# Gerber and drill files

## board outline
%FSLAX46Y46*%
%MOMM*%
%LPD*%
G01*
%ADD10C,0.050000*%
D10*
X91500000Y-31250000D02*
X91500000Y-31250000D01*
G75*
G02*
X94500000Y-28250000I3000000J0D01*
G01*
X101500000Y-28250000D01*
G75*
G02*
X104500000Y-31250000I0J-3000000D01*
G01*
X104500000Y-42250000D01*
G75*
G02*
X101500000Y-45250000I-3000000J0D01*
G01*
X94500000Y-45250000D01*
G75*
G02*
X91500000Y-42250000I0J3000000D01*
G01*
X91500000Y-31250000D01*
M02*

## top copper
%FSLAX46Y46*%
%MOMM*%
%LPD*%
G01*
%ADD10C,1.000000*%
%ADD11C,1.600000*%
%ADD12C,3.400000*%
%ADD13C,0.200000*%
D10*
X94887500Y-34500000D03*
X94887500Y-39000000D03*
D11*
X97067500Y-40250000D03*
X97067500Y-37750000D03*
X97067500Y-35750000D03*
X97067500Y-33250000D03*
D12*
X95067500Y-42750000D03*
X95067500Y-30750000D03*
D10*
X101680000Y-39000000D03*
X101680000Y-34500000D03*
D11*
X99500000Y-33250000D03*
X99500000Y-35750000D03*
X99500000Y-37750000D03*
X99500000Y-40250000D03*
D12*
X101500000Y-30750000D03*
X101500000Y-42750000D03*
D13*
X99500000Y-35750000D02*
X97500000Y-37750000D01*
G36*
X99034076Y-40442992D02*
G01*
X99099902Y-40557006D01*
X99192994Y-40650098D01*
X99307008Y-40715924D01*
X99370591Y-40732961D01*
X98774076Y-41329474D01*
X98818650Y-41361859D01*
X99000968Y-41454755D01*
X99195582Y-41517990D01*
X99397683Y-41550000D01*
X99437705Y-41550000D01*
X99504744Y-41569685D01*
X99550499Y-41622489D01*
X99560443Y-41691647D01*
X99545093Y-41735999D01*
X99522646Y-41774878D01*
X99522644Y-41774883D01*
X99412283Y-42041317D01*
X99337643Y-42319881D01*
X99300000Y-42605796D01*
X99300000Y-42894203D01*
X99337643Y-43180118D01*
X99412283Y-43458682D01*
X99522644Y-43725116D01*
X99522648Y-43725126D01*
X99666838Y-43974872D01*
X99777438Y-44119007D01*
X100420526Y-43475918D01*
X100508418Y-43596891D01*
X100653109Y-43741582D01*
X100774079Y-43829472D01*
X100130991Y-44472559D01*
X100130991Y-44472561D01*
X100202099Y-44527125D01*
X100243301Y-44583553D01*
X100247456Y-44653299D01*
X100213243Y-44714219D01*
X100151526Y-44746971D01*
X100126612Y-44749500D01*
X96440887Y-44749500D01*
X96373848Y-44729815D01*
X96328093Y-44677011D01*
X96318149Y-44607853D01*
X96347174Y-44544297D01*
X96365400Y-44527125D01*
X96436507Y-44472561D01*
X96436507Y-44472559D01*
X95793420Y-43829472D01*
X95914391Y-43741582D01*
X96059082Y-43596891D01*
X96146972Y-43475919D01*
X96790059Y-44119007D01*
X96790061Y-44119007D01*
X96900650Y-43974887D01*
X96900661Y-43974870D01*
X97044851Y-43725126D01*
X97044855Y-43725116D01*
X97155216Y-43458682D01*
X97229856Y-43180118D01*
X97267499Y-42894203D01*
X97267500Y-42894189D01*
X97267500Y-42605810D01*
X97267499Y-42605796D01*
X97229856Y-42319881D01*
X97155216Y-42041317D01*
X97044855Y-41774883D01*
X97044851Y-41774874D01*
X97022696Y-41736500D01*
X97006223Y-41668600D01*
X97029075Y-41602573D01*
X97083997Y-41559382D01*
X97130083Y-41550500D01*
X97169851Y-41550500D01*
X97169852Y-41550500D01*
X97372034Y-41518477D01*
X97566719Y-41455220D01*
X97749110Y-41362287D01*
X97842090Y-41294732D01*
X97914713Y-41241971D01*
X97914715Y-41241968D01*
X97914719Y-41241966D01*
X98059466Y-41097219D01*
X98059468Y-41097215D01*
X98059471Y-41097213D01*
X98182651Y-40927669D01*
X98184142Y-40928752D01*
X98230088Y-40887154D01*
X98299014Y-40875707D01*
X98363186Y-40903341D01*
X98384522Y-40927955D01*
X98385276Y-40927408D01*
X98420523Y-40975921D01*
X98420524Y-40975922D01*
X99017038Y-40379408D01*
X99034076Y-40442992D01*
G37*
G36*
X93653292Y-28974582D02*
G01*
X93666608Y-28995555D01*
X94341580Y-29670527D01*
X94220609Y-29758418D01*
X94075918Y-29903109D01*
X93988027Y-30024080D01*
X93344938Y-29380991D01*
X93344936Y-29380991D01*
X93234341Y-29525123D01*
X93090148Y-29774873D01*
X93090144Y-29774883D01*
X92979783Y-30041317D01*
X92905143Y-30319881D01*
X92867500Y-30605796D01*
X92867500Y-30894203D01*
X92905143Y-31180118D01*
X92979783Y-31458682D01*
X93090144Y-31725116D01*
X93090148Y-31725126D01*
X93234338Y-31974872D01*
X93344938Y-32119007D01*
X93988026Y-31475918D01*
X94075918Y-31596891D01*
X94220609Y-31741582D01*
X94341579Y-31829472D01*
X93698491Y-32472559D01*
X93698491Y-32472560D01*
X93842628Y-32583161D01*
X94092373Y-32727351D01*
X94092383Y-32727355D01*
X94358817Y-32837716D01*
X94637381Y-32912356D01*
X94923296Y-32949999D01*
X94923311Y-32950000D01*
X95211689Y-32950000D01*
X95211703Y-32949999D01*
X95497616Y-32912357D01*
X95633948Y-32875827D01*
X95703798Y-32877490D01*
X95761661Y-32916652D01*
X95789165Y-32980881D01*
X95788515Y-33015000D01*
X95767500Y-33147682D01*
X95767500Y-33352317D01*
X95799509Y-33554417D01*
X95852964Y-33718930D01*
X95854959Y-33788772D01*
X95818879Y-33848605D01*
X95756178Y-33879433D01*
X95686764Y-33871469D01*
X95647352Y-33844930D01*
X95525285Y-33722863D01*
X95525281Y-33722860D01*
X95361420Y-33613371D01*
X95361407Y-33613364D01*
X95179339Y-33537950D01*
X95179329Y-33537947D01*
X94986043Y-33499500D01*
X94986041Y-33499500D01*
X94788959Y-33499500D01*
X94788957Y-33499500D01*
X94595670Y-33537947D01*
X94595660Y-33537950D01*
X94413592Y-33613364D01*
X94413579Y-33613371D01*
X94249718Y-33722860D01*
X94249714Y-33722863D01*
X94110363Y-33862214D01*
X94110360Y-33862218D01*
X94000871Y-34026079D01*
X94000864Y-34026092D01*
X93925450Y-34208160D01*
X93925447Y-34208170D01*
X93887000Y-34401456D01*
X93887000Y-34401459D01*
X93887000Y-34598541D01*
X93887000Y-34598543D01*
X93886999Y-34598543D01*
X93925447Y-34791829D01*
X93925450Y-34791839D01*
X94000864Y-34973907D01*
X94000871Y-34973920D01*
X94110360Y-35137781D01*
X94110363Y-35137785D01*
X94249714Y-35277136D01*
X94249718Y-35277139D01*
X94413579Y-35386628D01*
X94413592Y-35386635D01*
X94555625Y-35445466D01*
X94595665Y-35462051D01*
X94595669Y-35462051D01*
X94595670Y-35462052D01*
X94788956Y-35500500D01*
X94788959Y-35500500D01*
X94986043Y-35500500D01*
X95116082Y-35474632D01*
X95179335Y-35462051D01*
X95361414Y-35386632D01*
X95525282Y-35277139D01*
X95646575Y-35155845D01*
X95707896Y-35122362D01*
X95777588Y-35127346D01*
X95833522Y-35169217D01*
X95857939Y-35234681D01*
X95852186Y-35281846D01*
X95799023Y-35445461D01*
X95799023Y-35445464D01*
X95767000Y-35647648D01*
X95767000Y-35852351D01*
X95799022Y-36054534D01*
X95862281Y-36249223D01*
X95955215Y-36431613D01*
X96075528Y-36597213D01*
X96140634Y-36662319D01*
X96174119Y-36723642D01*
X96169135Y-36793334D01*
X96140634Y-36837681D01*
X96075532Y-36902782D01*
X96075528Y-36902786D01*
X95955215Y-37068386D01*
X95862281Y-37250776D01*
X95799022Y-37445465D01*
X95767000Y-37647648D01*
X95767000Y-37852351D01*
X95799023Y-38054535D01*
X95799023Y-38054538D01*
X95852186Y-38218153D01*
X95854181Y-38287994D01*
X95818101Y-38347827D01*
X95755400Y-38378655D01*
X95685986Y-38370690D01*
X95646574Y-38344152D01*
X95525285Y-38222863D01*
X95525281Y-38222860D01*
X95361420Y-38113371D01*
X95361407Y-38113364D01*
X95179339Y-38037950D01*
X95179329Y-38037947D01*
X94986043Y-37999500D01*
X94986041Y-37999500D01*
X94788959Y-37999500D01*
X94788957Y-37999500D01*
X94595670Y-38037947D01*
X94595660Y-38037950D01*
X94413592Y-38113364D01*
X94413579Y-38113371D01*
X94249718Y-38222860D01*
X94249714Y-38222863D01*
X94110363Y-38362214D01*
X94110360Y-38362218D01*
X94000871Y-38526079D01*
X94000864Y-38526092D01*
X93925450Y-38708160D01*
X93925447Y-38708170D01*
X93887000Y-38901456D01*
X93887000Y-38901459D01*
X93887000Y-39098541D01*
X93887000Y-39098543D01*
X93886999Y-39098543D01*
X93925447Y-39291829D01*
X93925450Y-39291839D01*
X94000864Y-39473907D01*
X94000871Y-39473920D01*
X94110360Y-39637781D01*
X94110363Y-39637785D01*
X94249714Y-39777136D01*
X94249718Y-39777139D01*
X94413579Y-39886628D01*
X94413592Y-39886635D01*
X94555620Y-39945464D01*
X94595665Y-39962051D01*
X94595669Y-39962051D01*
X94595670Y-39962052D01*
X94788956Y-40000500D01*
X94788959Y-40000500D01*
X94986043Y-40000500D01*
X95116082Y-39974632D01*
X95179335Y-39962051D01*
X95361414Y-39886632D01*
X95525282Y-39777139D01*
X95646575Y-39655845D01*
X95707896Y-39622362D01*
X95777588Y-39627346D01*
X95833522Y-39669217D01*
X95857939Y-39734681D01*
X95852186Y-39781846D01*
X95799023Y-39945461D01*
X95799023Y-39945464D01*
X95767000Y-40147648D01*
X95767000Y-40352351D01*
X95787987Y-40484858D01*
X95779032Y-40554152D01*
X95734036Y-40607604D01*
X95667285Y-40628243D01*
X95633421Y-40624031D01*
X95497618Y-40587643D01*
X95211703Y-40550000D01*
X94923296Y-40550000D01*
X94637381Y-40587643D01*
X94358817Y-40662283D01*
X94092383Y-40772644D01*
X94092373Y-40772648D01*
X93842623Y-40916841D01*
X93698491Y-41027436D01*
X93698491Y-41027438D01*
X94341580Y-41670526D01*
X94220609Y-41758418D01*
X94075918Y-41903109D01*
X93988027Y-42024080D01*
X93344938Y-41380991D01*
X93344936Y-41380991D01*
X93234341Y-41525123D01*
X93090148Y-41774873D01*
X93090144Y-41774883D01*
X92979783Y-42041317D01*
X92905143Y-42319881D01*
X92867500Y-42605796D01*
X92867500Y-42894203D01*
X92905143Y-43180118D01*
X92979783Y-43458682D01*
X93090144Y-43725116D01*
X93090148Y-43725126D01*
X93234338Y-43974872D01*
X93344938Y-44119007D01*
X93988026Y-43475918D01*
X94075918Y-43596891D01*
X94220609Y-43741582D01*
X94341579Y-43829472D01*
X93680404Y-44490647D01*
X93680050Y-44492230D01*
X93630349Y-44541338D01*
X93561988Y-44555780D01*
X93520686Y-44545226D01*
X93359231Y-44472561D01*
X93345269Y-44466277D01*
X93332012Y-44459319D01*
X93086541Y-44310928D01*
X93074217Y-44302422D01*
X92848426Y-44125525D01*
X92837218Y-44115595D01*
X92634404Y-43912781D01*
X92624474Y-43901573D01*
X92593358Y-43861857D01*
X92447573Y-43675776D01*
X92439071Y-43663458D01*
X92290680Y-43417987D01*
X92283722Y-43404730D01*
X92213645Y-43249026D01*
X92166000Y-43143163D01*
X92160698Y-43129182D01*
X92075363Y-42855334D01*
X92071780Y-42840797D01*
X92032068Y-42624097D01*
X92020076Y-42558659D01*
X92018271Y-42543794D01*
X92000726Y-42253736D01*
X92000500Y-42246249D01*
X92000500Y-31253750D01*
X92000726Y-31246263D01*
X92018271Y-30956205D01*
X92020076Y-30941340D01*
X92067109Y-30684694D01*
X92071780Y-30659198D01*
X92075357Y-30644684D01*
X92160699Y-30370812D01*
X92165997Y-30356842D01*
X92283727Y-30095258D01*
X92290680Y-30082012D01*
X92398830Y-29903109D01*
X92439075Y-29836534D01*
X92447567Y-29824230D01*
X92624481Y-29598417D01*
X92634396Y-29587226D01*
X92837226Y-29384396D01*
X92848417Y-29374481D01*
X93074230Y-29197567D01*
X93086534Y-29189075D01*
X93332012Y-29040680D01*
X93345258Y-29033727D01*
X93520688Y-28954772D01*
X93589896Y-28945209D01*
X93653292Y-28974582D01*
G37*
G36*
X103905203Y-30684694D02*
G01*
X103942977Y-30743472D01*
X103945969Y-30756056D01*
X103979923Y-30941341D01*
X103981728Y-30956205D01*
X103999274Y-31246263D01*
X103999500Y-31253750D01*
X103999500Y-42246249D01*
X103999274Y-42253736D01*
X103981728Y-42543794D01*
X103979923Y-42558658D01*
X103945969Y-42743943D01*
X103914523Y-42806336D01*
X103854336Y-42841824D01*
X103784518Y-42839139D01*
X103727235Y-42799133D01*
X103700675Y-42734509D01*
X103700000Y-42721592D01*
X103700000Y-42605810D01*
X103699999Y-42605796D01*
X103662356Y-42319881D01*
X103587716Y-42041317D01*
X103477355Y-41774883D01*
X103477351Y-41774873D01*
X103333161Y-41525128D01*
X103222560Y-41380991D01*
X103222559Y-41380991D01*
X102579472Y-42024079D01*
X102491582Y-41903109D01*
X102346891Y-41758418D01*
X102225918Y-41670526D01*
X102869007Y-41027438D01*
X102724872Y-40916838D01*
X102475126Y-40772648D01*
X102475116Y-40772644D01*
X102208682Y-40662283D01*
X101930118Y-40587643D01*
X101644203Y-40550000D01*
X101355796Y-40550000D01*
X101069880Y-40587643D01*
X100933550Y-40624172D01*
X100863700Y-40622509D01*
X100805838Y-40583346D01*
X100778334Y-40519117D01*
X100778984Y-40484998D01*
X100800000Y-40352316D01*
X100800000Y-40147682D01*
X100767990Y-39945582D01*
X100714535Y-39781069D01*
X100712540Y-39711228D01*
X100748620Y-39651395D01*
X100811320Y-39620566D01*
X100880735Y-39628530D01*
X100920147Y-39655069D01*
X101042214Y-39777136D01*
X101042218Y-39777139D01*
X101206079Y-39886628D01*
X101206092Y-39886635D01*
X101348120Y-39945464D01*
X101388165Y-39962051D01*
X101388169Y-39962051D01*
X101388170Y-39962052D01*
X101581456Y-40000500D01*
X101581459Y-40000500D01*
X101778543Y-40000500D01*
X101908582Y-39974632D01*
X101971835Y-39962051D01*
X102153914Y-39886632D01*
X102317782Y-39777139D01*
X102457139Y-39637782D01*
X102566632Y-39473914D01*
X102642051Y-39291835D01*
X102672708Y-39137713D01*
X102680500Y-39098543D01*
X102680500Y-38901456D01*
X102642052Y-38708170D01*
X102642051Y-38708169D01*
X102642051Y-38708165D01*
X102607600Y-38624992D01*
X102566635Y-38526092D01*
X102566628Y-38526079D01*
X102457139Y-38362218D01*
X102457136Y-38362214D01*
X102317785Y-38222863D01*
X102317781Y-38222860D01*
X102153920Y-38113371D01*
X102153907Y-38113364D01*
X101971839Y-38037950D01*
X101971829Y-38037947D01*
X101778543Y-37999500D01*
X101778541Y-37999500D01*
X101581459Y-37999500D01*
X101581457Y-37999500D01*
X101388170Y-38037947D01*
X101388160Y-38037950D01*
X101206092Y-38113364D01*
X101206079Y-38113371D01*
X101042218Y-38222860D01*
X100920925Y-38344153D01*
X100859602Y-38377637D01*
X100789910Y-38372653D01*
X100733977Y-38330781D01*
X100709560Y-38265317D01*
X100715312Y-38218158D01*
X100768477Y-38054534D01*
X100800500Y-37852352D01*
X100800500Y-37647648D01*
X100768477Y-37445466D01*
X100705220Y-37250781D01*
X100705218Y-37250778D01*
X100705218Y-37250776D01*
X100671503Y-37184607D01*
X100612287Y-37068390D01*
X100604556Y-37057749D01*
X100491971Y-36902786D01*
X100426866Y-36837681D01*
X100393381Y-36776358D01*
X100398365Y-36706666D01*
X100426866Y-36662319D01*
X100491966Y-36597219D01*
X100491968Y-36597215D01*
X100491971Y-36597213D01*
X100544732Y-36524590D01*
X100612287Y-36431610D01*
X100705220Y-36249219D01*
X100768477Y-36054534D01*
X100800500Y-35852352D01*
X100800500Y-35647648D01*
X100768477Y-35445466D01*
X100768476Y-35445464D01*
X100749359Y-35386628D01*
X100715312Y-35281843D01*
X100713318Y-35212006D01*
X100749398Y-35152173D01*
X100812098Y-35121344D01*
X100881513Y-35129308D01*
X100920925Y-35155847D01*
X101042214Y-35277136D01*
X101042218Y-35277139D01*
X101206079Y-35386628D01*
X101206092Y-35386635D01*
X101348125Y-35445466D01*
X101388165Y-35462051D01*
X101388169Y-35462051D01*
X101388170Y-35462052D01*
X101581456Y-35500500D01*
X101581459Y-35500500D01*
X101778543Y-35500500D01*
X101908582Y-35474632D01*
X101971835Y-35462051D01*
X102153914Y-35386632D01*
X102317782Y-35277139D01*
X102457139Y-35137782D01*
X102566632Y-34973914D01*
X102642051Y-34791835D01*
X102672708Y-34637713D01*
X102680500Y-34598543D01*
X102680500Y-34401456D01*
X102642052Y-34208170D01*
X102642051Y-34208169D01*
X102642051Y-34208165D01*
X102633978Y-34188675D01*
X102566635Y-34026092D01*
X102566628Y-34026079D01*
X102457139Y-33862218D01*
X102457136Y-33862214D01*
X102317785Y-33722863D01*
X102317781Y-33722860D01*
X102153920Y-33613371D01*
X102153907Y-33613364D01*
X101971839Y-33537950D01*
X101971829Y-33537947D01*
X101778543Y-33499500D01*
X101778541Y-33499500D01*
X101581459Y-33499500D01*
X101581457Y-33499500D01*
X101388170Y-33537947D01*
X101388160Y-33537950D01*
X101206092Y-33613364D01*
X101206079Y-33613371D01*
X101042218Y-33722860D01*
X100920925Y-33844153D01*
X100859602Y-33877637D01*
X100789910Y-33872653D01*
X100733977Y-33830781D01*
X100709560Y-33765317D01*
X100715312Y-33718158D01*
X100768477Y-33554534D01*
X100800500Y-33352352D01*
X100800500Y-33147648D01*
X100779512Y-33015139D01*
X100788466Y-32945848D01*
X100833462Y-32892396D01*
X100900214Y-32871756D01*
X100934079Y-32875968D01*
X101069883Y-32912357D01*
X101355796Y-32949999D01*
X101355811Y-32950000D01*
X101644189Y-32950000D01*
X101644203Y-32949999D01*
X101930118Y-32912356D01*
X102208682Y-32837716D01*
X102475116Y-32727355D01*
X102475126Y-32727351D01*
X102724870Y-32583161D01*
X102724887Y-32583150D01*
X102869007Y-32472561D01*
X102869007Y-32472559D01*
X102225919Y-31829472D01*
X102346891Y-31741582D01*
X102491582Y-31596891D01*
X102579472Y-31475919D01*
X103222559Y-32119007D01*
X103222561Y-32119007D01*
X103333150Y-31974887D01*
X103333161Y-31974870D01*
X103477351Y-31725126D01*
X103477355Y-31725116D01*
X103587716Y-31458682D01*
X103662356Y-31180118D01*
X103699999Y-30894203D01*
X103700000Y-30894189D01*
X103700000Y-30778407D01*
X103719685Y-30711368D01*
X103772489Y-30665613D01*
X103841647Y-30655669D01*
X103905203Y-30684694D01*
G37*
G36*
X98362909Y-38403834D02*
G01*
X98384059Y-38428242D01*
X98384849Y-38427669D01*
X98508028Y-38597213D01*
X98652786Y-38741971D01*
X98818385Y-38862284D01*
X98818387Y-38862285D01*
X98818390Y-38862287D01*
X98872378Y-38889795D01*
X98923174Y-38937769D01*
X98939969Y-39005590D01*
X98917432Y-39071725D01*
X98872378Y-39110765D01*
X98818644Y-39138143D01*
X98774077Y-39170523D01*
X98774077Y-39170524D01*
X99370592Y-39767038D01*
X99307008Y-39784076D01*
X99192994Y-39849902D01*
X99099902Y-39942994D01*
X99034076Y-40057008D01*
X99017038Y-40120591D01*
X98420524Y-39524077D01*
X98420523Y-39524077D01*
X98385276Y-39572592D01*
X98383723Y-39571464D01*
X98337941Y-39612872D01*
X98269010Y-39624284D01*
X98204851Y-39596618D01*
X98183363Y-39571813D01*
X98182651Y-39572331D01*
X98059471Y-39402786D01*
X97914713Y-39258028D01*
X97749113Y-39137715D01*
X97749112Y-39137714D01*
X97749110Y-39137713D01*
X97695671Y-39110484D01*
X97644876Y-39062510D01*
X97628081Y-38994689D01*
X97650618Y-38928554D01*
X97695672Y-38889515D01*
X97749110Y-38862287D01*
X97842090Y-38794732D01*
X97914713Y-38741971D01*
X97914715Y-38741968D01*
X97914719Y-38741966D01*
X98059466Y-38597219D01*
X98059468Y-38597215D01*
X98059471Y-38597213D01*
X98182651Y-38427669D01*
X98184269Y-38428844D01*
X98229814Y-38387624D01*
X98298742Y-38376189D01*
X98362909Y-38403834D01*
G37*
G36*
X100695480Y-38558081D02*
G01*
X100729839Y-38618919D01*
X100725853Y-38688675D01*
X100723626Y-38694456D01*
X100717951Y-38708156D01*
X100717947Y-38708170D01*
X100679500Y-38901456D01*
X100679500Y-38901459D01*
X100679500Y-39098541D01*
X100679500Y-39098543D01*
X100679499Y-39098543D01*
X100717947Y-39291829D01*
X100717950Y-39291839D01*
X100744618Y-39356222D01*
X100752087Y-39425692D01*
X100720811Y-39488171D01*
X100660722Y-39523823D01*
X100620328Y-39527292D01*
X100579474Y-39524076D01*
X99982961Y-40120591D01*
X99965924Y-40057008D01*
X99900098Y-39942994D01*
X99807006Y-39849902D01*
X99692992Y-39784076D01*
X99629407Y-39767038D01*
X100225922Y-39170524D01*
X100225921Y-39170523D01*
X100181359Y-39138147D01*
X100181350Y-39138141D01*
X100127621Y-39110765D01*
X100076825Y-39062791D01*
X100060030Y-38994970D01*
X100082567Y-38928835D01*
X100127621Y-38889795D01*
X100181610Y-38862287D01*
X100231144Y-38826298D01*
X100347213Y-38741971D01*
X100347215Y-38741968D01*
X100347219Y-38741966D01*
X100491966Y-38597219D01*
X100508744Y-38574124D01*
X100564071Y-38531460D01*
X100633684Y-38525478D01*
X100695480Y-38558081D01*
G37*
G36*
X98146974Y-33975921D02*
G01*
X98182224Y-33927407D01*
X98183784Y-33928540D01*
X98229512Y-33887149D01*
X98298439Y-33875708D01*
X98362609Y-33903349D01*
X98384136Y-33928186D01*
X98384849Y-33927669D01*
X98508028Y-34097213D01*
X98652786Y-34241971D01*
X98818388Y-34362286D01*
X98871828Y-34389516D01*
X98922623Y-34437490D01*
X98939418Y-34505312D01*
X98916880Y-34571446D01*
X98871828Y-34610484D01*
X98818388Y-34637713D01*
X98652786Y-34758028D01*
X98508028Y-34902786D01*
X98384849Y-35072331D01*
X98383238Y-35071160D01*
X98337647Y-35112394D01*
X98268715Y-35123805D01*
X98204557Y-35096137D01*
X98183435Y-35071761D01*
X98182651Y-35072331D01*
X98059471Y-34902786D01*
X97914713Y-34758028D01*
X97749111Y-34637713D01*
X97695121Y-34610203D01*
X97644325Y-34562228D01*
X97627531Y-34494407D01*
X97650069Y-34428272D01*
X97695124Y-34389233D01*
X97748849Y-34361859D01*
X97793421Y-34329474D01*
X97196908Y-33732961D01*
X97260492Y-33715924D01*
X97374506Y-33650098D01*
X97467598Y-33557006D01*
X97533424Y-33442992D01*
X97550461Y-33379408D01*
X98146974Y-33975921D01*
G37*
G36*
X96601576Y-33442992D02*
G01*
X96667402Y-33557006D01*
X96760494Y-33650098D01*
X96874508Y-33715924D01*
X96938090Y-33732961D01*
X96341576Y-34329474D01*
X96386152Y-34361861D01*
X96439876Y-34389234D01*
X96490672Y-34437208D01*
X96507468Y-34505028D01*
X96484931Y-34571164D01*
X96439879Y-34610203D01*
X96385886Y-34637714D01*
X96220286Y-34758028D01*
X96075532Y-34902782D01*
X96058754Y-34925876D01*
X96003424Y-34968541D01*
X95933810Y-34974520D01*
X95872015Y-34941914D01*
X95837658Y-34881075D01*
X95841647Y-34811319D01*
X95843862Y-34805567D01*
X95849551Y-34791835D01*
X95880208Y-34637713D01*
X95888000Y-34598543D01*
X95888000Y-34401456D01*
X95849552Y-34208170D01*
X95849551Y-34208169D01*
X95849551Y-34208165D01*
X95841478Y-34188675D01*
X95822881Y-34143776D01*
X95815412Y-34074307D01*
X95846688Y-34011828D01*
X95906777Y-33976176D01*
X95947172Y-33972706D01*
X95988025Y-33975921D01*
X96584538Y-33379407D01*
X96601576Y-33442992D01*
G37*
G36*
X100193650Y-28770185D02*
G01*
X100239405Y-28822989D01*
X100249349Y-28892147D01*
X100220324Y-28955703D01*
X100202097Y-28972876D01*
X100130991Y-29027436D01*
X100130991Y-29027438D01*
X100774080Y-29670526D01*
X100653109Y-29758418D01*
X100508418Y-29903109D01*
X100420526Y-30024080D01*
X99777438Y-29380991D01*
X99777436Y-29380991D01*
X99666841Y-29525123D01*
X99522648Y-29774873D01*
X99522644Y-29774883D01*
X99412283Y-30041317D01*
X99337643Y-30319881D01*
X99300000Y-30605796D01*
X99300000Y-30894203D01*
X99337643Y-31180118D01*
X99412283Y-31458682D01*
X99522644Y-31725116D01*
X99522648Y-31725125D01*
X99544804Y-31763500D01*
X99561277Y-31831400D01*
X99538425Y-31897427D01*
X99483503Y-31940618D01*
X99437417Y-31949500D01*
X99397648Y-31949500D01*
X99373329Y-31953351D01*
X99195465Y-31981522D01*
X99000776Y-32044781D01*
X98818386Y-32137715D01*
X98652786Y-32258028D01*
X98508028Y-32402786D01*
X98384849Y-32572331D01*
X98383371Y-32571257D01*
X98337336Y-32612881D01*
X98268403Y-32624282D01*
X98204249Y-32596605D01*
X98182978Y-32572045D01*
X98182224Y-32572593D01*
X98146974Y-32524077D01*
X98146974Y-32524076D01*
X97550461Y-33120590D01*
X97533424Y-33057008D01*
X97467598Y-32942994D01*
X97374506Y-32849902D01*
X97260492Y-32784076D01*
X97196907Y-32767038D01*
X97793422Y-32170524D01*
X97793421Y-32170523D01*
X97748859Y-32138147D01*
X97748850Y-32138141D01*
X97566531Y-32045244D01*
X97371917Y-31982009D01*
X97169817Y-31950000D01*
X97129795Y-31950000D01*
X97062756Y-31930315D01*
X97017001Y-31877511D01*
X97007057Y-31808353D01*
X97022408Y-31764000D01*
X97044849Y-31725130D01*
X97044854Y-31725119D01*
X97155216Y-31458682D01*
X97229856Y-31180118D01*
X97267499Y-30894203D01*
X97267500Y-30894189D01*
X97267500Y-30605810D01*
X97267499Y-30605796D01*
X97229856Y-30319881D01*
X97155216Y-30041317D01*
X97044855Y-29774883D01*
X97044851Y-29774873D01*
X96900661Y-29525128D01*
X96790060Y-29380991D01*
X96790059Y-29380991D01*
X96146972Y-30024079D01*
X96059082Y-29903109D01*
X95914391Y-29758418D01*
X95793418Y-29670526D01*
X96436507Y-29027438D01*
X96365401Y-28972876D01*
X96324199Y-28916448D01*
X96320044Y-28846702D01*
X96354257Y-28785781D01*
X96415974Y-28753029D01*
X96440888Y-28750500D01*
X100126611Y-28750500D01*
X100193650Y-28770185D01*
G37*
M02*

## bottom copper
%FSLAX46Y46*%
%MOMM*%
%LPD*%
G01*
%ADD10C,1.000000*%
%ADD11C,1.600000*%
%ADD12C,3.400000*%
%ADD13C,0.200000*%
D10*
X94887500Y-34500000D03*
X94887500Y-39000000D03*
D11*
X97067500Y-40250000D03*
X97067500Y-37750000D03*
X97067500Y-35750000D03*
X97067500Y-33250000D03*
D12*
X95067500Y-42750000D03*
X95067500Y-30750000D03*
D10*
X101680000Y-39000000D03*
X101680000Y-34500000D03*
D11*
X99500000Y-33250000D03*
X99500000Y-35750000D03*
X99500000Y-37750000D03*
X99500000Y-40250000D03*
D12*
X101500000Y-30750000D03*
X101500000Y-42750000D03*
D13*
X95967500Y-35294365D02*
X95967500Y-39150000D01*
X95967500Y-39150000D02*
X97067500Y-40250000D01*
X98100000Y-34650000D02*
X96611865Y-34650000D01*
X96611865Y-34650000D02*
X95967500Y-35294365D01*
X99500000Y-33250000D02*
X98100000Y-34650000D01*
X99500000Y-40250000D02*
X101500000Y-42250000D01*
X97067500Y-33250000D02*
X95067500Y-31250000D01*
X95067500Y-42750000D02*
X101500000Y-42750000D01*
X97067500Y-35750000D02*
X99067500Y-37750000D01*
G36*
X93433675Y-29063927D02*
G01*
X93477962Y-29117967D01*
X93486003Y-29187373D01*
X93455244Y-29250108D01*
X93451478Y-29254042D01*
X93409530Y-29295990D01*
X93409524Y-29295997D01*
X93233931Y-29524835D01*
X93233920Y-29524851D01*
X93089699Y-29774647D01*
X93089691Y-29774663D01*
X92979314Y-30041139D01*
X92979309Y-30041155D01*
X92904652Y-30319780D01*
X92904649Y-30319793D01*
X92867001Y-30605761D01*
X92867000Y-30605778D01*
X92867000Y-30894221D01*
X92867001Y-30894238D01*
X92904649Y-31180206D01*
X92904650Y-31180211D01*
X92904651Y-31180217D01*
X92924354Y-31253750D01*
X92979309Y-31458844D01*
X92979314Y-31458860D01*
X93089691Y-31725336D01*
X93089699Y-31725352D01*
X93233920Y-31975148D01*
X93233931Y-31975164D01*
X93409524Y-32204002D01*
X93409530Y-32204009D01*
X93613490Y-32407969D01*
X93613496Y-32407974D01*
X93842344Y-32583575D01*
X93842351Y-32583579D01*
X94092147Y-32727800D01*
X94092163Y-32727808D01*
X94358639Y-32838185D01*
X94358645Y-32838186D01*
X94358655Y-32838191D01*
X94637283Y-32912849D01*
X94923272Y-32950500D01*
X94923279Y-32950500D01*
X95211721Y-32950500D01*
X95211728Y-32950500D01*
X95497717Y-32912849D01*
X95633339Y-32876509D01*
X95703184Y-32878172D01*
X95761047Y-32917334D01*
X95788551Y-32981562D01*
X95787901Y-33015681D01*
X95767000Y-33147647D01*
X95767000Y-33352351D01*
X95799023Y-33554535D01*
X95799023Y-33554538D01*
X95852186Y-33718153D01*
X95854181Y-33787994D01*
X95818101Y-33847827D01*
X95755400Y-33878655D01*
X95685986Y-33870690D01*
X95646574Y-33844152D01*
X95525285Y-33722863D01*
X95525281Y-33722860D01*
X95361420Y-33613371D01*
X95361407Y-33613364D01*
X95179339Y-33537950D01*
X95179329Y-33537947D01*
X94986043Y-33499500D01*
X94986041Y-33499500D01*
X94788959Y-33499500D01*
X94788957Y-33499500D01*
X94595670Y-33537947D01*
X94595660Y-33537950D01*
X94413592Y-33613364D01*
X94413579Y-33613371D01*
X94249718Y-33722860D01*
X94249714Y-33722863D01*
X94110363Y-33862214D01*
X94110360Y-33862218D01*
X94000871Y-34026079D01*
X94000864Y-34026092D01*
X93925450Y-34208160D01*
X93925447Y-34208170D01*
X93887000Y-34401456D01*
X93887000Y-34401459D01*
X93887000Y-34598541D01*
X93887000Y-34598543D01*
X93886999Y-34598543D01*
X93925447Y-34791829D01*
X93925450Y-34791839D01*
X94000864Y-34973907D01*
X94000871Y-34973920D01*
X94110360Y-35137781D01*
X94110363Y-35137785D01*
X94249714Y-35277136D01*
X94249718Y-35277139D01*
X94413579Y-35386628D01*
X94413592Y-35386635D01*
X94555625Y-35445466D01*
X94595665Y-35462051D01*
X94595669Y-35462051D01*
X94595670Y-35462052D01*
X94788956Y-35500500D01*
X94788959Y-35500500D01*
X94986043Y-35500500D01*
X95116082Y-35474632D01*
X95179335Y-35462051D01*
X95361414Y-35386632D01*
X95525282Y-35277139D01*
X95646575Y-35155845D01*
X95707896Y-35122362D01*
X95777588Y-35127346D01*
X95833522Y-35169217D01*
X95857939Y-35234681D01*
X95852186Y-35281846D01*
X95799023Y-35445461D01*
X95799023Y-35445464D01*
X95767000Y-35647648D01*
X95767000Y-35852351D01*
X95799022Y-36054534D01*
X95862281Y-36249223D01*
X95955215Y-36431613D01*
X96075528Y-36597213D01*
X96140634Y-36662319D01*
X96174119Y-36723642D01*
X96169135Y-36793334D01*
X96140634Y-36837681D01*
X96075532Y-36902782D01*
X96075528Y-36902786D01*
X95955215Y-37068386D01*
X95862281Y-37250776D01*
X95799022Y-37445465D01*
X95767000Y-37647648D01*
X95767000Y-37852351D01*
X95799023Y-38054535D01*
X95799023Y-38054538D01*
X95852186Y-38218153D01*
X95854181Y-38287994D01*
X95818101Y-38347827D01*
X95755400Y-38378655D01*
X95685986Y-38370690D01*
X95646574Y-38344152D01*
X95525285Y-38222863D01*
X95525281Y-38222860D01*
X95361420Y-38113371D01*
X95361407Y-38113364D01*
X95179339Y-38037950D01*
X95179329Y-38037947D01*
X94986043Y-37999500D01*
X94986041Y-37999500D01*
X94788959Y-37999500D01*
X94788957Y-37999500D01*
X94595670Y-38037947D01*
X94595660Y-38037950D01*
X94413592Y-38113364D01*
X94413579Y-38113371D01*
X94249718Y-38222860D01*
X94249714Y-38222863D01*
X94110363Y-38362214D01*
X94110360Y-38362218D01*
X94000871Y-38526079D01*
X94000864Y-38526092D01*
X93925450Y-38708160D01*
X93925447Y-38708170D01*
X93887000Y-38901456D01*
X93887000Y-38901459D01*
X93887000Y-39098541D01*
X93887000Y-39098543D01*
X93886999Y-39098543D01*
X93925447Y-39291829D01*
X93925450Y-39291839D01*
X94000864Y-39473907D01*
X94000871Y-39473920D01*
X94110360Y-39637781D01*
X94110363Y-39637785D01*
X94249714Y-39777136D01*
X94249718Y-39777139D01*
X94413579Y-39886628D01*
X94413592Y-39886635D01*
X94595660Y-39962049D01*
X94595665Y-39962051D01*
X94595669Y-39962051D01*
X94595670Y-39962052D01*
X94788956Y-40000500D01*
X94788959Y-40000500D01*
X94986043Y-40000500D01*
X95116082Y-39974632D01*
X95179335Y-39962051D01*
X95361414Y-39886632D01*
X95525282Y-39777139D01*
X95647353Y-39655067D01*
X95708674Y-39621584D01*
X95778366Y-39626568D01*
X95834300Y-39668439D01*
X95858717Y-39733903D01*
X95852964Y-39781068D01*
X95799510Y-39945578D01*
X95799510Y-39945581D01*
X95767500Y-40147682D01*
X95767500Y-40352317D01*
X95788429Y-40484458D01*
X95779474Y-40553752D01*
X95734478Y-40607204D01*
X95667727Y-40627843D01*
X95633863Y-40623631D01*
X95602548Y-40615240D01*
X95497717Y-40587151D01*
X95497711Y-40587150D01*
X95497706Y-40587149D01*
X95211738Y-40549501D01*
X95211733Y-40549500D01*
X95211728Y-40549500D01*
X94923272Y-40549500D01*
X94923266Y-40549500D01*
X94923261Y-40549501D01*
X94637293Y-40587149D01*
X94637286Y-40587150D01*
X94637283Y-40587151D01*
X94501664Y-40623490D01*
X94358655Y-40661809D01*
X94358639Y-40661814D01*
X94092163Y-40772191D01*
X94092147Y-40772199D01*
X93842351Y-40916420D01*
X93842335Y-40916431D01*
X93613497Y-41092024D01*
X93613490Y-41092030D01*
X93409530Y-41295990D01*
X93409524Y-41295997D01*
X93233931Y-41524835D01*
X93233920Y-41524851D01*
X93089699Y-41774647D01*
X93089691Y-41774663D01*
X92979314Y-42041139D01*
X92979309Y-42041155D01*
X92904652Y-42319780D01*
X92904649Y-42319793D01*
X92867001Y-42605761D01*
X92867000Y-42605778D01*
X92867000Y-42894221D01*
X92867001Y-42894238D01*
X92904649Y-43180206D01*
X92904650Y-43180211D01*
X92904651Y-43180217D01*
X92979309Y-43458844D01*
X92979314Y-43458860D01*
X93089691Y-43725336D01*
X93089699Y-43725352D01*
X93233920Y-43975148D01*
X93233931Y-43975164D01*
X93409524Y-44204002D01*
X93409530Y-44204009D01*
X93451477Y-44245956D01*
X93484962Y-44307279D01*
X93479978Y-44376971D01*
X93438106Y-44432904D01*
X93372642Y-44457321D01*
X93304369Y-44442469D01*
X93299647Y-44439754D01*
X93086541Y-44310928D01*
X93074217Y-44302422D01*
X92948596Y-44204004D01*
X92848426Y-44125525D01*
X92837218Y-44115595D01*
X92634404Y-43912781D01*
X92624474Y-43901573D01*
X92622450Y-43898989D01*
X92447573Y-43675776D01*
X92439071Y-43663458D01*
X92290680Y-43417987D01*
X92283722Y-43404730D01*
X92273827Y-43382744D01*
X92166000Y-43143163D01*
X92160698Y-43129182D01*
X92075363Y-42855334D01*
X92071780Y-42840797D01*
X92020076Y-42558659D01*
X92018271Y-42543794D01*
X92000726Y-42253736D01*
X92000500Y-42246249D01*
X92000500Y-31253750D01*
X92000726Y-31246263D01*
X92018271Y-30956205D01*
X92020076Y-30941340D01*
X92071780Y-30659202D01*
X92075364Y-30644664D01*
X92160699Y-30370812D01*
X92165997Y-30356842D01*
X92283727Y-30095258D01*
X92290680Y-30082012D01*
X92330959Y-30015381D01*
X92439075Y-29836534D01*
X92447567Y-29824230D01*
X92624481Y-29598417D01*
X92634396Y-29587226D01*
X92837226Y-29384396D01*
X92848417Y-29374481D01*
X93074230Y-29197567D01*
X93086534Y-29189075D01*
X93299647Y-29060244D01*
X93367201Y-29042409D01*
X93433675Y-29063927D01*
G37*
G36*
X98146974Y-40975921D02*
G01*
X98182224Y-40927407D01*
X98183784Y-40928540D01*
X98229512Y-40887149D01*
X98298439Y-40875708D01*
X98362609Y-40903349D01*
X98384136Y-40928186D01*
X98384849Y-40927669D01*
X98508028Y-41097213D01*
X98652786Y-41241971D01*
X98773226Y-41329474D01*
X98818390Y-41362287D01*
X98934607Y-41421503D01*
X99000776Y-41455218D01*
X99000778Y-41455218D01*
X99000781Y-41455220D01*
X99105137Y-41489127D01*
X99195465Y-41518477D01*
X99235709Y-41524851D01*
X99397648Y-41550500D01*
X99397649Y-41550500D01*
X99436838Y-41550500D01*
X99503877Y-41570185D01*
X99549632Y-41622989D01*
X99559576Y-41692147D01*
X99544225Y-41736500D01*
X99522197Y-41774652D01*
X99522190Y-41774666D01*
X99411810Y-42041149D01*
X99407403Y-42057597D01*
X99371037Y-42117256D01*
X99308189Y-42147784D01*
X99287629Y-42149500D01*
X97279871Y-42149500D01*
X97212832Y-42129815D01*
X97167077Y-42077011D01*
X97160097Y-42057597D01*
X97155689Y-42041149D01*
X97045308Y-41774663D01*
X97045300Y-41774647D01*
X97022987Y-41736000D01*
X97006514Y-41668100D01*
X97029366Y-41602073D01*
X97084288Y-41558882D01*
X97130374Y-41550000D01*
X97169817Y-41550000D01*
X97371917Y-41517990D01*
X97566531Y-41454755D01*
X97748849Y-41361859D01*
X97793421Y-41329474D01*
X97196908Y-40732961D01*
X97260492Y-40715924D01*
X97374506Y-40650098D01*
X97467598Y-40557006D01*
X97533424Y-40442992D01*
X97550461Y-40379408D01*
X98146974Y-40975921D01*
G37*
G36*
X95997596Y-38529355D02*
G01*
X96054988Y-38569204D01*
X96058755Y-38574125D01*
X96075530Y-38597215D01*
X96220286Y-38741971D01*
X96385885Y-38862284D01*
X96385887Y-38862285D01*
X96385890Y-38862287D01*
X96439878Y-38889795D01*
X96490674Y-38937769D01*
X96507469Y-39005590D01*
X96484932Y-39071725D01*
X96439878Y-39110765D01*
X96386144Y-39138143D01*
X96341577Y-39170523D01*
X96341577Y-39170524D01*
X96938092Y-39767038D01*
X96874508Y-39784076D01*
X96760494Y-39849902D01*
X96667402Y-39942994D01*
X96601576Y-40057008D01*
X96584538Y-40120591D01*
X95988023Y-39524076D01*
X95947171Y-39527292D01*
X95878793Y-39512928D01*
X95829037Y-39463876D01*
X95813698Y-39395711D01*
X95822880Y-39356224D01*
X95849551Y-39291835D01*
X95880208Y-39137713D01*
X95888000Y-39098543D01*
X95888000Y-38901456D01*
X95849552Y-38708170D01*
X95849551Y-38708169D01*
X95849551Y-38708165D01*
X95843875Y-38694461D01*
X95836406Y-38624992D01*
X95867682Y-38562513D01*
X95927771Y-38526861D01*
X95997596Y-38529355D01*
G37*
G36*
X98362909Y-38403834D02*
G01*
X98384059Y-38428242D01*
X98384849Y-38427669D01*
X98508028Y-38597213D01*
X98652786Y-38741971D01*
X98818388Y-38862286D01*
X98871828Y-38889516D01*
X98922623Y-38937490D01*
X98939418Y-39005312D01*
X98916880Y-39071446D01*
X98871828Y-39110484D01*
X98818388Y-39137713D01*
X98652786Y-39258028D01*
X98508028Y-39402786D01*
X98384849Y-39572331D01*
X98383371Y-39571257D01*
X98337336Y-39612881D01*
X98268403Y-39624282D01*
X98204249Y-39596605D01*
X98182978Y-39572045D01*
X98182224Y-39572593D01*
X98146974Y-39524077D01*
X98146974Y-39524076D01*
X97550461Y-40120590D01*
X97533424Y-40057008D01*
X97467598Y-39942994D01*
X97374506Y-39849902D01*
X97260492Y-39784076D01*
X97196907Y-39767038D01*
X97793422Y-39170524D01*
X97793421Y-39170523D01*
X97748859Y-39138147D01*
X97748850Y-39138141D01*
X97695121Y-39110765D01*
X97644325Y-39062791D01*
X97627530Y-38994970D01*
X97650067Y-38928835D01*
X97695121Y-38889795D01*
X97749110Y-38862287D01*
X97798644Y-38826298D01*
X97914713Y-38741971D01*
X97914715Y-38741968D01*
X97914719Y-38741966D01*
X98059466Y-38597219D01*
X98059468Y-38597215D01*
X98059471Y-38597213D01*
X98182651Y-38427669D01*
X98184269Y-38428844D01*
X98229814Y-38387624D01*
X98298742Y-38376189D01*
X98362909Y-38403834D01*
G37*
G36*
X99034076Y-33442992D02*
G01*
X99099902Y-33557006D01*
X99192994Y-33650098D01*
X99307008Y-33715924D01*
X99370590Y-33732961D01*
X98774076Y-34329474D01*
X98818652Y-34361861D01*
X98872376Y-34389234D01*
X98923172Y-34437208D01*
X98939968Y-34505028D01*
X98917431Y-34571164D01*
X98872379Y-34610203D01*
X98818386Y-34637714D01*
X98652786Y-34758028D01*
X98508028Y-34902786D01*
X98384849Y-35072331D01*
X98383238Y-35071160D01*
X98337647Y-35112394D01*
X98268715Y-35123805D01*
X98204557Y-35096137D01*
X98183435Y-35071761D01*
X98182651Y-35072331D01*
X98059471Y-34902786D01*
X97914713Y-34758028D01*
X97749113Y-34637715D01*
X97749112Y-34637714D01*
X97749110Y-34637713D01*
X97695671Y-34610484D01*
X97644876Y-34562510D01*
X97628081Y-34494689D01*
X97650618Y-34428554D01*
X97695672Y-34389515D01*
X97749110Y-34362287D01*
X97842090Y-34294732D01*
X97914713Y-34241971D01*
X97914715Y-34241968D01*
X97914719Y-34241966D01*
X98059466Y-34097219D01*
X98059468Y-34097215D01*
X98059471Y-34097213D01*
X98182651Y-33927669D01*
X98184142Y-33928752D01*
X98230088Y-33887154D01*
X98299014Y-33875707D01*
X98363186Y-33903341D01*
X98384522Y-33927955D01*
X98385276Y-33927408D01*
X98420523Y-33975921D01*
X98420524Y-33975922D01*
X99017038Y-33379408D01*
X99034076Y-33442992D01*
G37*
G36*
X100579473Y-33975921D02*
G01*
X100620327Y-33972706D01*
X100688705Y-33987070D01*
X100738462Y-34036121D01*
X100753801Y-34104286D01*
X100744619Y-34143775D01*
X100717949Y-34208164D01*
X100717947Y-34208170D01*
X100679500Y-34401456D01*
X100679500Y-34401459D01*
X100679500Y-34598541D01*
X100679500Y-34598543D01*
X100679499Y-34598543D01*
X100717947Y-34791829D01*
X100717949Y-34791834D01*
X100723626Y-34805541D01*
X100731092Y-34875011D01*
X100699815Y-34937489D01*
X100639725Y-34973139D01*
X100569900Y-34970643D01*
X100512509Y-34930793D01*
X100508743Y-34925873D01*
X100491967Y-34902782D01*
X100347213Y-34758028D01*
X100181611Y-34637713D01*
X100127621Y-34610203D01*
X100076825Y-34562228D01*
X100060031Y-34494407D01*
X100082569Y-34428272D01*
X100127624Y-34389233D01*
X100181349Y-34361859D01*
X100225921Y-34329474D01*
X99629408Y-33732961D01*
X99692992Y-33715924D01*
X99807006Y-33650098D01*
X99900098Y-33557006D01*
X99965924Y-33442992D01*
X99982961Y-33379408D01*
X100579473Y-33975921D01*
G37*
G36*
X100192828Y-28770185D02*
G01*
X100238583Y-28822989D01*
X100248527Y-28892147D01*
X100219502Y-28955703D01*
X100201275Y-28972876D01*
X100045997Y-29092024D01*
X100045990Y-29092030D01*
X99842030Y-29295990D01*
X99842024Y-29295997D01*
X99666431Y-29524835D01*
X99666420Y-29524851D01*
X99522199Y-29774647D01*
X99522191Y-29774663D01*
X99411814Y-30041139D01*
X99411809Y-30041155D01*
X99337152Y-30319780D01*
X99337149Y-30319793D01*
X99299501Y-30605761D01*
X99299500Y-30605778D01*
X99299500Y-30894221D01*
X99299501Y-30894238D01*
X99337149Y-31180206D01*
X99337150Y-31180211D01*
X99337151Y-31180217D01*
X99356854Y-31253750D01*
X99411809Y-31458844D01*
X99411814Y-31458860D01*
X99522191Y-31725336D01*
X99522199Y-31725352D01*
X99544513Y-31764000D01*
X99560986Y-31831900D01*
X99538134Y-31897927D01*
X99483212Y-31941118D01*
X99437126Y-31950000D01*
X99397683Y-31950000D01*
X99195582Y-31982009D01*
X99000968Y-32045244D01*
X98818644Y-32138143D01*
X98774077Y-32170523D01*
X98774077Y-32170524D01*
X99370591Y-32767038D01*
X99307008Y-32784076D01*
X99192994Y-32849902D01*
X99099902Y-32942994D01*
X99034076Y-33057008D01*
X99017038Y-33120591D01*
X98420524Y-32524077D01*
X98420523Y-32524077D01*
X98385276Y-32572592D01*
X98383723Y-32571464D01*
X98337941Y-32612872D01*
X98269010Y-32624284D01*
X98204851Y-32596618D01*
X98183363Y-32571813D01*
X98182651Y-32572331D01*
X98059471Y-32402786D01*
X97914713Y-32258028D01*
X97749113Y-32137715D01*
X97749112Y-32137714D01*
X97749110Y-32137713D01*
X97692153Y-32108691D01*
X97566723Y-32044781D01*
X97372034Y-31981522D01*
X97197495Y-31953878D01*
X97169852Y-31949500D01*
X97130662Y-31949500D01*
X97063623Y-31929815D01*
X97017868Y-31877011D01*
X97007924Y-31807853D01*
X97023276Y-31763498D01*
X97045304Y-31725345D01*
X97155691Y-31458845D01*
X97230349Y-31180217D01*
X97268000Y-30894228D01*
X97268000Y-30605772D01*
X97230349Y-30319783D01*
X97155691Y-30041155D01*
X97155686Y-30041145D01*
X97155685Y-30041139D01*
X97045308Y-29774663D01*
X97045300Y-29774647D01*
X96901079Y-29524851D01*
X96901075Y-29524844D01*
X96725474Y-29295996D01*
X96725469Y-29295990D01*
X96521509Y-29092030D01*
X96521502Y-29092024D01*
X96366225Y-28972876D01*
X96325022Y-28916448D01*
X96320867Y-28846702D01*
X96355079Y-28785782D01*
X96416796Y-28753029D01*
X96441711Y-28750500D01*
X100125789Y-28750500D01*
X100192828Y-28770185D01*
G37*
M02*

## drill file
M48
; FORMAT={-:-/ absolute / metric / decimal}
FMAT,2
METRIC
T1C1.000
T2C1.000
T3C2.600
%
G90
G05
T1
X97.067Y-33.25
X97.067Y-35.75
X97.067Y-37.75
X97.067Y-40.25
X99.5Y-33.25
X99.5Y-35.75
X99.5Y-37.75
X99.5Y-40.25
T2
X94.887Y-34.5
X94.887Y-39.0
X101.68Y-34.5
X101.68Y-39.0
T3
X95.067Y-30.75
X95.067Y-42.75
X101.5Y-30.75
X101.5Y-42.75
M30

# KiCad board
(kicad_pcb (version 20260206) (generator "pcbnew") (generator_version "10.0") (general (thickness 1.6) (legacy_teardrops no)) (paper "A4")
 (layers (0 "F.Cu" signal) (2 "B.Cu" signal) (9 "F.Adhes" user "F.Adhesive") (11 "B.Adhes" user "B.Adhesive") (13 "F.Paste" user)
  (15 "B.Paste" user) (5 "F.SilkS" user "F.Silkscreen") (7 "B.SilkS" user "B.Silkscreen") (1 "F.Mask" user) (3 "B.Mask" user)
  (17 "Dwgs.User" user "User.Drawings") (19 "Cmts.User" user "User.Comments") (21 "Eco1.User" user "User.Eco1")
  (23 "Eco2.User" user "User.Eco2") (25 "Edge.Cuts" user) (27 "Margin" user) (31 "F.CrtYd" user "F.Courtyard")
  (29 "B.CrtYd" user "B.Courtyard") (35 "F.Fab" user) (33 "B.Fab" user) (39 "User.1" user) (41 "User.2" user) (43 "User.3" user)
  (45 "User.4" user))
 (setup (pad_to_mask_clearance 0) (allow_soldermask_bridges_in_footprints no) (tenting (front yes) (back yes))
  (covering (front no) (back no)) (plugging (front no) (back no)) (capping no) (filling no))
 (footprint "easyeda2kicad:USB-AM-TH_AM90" (layer "F.Cu") (at 96.0675 36.75 -90)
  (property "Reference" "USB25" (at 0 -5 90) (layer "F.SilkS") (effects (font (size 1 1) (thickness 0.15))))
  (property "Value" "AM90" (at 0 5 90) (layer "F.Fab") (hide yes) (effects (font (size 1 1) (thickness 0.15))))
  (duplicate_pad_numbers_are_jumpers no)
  (pad "" thru_hole circle (at -2.25 1.18 270) (size 1 1) (drill 1) (layers "*.Cu" "*.Mask") (remove_unused_layers no))
  (pad "" thru_hole circle (at 2.25 1.18 270) (size 1 1) (drill 1) (layers "*.Cu" "*.Mask") (remove_unused_layers no))
  (pad "1" thru_hole circle (at 3.5 -1 180) (size 1.6 1.6) (drill 0.999998) (layers "*.Cu" "*.Mask") (remove_unused_layers no)
   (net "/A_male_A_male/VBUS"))
  (pad "2" thru_hole circle (at 1 -1 180) (size 1.6 1.6) (drill 0.999998) (layers "*.Cu" "*.Mask") (remove_unused_layers no)
   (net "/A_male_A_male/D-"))
  (pad "3" thru_hole circle (at -1 -1 180) (size 1.6 1.6) (drill 0.999998) (layers "*.Cu" "*.Mask") (remove_unused_layers no)
   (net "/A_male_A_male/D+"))
  (pad "4" thru_hole circle (at -3.5 -1 180) (size 1.6 1.6) (drill 0.999998) (layers "*.Cu" "*.Mask") (remove_unused_layers no)
   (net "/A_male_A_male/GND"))
  (pad "MH1" thru_hole circle (at 6 1 180) (size 3.4 3.4) (drill 2.599994) (layers "*.Cu" "*.Mask") (remove_unused_layers no)
   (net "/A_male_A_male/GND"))
  (pad "MH2" thru_hole circle (at -6 1 180) (size 3.4 3.4) (drill 2.599994) (layers "*.Cu" "*.Mask") (remove_unused_layers no)
   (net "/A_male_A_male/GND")))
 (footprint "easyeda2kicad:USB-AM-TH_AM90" (layer "F.Cu") (at 100.5 36.75 90)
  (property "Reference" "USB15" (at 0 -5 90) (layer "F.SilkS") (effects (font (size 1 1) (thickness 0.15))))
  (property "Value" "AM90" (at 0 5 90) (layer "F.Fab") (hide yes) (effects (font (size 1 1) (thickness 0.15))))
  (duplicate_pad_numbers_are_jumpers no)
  (pad "" thru_hole circle (at -2.25 1.18 90) (size 1 1) (drill 1) (layers "*.Cu" "*.Mask") (remove_unused_layers no))
  (pad "" thru_hole circle (at 2.25 1.18 90) (size 1 1) (drill 1) (layers "*.Cu" "*.Mask") (remove_unused_layers no))
  (pad "1" thru_hole circle (at 3.5 -1) (size 1.6 1.6) (drill 0.999998) (layers "*.Cu" "*.Mask") (remove_unused_layers no)
   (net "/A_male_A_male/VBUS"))
  (pad "2" thru_hole circle (at 1 -1) (size 1.6 1.6) (drill 0.999998) (layers "*.Cu" "*.Mask") (remove_unused_layers no)
   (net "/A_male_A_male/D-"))
  (pad "3" thru_hole circle (at -1 -1) (size 1.6 1.6) (drill 0.999998) (layers "*.Cu" "*.Mask") (remove_unused_layers no)
   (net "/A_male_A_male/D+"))
  (pad "4" thru_hole circle (at -3.5 -1) (size 1.6 1.6) (drill 0.999998) (layers "*.Cu" "*.Mask") (remove_unused_layers no)
   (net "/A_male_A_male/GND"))
  (pad "MH1" thru_hole circle (at 6 1) (size 3.4 3.4) (drill 2.599994) (layers "*.Cu" "*.Mask") (remove_unused_layers no)
   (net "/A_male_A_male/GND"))
  (pad "MH2" thru_hole circle (at -6 1) (size 3.4 3.4) (drill 2.599994) (layers "*.Cu" "*.Mask") (remove_unused_layers no)
   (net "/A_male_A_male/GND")))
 (gr_rect (start 91.5 28.25) (end 104.5 45.25) (radius 3) (stroke (width 0.05) (type solid)) (fill no) (layer "Edge.Cuts"))
 (segment (start 95.9675 35.294365) (end 95.9675 39.15) (width 0.2) (layer "B.Cu") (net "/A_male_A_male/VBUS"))
 (segment (start 95.9675 39.15) (end 97.0675 40.25) (width 0.2) (layer "B.Cu") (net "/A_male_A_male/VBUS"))
 (segment (start 98.1 34.65) (end 96.611865 34.65) (width 0.2) (layer "B.Cu") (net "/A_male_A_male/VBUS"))
 (segment (start 96.611865 34.65) (end 95.9675 35.294365) (width 0.2) (layer "B.Cu") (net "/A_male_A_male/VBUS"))
 (segment (start 99.5 33.25) (end 98.1 34.65) (width 0.2) (layer "B.Cu") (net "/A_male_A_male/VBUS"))
 (segment (start 99.5 35.75) (end 97.5 37.75) (width 0.2) (layer "F.Cu") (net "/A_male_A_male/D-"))
 (segment (start 99.5 40.25) (end 101.5 42.25) (width 0.2) (layer "B.Cu") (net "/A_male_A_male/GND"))
 (segment (start 97.0675 33.25) (end 95.0675 31.25) (width 0.2) (layer "B.Cu") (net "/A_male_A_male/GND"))
 (segment (start 95.0675 42.75) (end 101.5 42.75) (width 0.2) (layer "B.Cu") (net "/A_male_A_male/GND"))
 (segment (start 97.0675 35.75) (end 99.0675 37.75) (width 0.2) (layer "B.Cu") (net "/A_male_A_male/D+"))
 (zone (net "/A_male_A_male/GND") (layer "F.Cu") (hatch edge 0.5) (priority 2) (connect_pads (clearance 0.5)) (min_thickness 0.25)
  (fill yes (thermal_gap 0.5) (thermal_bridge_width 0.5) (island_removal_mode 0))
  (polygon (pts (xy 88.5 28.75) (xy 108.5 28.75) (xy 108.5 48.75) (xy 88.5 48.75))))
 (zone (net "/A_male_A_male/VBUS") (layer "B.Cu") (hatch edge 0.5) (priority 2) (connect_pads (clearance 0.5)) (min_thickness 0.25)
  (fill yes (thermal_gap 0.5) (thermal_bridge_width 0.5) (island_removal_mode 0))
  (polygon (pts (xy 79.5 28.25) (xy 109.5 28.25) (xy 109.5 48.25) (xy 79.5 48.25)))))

